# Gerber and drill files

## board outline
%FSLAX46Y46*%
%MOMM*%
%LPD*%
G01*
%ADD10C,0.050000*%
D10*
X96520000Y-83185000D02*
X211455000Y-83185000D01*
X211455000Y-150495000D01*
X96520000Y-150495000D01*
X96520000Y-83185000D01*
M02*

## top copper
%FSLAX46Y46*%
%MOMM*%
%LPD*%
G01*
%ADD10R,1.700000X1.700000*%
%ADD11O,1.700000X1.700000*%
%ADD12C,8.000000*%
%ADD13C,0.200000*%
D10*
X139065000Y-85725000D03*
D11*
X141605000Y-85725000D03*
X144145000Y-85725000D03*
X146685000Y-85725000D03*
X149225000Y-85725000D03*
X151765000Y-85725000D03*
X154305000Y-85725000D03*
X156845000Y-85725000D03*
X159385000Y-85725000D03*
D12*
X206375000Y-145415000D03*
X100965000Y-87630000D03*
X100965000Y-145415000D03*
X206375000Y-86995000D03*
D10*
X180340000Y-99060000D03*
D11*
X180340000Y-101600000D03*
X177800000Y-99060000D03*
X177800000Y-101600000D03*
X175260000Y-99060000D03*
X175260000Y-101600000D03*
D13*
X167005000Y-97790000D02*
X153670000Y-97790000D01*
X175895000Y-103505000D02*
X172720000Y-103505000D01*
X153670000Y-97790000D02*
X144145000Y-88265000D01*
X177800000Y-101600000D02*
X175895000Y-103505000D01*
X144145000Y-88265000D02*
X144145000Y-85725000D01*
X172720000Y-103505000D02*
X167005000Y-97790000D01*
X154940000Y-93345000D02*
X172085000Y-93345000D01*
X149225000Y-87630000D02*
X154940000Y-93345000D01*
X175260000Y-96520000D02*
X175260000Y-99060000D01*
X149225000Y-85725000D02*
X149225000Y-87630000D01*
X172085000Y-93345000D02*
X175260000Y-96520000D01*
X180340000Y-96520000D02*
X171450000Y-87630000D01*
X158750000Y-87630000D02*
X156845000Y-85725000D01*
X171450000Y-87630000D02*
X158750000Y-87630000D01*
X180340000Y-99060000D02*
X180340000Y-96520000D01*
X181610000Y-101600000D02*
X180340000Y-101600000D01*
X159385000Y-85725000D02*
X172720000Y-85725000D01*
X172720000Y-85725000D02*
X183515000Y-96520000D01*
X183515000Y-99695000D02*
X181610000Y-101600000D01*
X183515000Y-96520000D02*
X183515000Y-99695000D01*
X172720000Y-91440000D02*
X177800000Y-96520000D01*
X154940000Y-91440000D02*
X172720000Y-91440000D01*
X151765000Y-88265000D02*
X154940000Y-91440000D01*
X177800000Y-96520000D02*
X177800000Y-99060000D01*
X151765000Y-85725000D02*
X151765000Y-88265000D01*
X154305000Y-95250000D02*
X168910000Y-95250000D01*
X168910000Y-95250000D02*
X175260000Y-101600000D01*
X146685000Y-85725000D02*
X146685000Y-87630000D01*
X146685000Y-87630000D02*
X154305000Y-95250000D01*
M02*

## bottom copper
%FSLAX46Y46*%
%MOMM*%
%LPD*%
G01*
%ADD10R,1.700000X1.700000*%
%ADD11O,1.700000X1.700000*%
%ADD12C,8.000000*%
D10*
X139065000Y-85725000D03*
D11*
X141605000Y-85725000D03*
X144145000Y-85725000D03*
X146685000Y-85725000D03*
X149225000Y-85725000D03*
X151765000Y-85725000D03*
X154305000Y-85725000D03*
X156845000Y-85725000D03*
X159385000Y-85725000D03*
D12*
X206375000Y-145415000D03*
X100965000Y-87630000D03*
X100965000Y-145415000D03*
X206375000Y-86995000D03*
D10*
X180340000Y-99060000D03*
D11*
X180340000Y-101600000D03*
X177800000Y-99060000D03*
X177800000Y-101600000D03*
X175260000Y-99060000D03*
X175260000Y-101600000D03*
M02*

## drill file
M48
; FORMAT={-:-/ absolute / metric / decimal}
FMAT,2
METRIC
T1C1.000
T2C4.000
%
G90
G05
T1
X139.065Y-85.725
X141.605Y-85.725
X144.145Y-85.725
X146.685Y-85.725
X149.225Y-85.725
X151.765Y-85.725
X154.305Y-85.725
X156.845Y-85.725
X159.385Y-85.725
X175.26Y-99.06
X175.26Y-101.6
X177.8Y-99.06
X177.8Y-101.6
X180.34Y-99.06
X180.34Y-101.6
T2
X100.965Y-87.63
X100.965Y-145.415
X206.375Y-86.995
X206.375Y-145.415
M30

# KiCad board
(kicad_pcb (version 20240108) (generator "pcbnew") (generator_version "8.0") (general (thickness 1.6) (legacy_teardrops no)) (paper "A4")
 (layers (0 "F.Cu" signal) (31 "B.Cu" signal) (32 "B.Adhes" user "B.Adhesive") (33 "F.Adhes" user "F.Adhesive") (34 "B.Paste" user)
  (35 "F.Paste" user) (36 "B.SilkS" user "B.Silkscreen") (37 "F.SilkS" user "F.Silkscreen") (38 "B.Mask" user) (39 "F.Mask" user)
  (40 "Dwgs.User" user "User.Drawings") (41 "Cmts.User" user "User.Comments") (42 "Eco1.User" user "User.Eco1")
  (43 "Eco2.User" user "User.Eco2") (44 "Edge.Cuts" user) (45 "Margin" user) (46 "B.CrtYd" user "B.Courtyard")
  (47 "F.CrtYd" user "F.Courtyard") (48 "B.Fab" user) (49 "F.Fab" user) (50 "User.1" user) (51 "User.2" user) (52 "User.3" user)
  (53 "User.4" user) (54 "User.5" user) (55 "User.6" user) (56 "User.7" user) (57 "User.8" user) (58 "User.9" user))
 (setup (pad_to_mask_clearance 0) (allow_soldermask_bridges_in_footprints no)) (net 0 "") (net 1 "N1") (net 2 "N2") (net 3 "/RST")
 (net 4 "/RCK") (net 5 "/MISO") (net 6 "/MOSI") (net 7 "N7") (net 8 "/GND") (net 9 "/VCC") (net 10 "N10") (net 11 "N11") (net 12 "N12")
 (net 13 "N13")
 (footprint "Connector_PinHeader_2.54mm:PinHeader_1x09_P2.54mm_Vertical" (layer "F.Cu") (at 139.065 85.725 90)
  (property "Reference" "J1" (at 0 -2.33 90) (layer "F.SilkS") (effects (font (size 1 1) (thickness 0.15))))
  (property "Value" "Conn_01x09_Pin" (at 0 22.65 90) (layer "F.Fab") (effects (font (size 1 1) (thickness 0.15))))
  (pad "1" thru_hole rect (at 0 0 90) (size 1.7 1.7) (drill 1) (layers "*.Cu" "*.Mask") (remove_unused_layers no) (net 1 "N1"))
  (pad "2" thru_hole oval (at 0 2.54 90) (size 1.7 1.7) (drill 1) (layers "*.Cu" "*.Mask") (remove_unused_layers no) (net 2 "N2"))
  (pad "3" thru_hole oval (at 0 5.08 90) (size 1.7 1.7) (drill 1) (layers "*.Cu" "*.Mask") (remove_unused_layers no) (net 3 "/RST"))
  (pad "4" thru_hole oval (at 0 7.62 90) (size 1.7 1.7) (drill 1) (layers "*.Cu" "*.Mask") (remove_unused_layers no) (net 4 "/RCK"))
  (pad "5" thru_hole oval (at 0 10.16 90) (size 1.7 1.7) (drill 1) (layers "*.Cu" "*.Mask") (remove_unused_layers no) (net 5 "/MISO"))
  (pad "6" thru_hole oval (at 0 12.7 90) (size 1.7 1.7) (drill 1) (layers "*.Cu" "*.Mask") (remove_unused_layers no) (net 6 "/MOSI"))
  (pad "7" thru_hole oval (at 0 15.24 90) (size 1.7 1.7) (drill 1) (layers "*.Cu" "*.Mask") (remove_unused_layers no) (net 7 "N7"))
  (pad "8" thru_hole oval (at 0 17.78 90) (size 1.7 1.7) (drill 1) (layers "*.Cu" "*.Mask") (remove_unused_layers no) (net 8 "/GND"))
  (pad "9" thru_hole oval (at 0 20.32 90) (size 1.7 1.7) (drill 1) (layers "*.Cu" "*.Mask") (remove_unused_layers no) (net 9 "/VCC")))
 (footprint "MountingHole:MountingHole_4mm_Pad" (layer "F.Cu") (at 206.375 145.415 90)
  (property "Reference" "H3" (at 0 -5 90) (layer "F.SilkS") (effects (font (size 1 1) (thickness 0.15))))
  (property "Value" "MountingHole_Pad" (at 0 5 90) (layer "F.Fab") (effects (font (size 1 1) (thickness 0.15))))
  (pad "1" thru_hole circle (at 0 0 90) (size 8 8) (drill 4) (layers "*.Cu" "*.Mask") (remove_unused_layers no) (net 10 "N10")))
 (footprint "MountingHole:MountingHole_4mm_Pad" (layer "F.Cu") (at 100.965 87.63 90)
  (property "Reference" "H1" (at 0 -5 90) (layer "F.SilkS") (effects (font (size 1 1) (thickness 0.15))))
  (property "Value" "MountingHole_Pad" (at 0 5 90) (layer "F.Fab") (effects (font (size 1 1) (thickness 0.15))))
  (pad "1" thru_hole circle (at 0 0 90) (size 8 8) (drill 4) (layers "*.Cu" "*.Mask") (remove_unused_layers no) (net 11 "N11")))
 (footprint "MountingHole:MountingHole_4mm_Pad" (layer "F.Cu") (at 100.965 145.415 90)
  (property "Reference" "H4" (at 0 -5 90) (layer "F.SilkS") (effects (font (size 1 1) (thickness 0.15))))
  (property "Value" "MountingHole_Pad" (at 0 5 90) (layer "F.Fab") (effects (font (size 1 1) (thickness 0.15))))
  (pad "1" thru_hole circle (at 0 0 90) (size 8 8) (drill 4) (layers "*.Cu" "*.Mask") (remove_unused_layers no) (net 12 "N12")))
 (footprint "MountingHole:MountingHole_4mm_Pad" (layer "F.Cu") (at 206.375 86.995 90)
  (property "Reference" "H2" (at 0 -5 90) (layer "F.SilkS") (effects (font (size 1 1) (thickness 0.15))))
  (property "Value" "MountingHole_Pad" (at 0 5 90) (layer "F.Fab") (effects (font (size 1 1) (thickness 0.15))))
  (pad "1" thru_hole circle (at 0 0 90) (size 8 8) (drill 4) (layers "*.Cu" "*.Mask") (remove_unused_layers no) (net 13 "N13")))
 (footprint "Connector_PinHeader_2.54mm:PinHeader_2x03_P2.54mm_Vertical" (layer "F.Cu") (at 180.34 99.06 -90)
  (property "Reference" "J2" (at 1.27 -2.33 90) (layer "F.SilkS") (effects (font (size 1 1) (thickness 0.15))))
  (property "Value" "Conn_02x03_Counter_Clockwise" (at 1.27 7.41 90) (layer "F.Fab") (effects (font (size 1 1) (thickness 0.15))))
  (pad "1" thru_hole rect (at 0 0 270) (size 1.7 1.7) (drill 1) (layers "*.Cu" "*.Mask") (remove_unused_layers no) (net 8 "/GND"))
  (pad "2" thru_hole oval (at 2.54 0 270) (size 1.7 1.7) (drill 1) (layers "*.Cu" "*.Mask") (remove_unused_layers no) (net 9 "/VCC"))
  (pad "3" thru_hole oval (at 0 2.54 270) (size 1.7 1.7) (drill 1) (layers "*.Cu" "*.Mask") (remove_unused_layers no) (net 6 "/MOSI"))
  (pad "4" thru_hole oval (at 2.54 2.54 270) (size 1.7 1.7) (drill 1) (layers "*.Cu" "*.Mask") (remove_unused_layers no) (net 3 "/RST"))
  (pad "5" thru_hole oval (at 0 5.08 270) (size 1.7 1.7) (drill 1) (layers "*.Cu" "*.Mask") (remove_unused_layers no) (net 5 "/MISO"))
  (pad "6" thru_hole oval (at 2.54 5.08 270) (size 1.7 1.7) (drill 1) (layers "*.Cu" "*.Mask") (remove_unused_layers no) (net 4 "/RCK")))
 (gr_rect (start 96.52 83.185) (end 211.455 150.495) (stroke (width 0.05) (type default)) (fill none) (layer "Edge.Cuts"))
 (segment (start 167.005 97.79) (end 153.67 97.79) (width 0.2) (layer "F.Cu") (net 3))
 (segment (start 175.895 103.505) (end 172.72 103.505) (width 0.2) (layer "F.Cu") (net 3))
 (segment (start 153.67 97.79) (end 144.145 88.265) (width 0.2) (layer "F.Cu") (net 3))
 (segment (start 177.8 101.6) (end 175.895 103.505) (width 0.2) (layer "F.Cu") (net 3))
 (segment (start 144.145 88.265) (end 144.145 85.725) (width 0.2) (layer "F.Cu") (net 3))
 (segment (start 172.72 103.505) (end 167.005 97.79) (width 0.2) (layer "F.Cu") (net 3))
 (segment (start 154.94 93.345) (end 172.085 93.345) (width 0.2) (layer "F.Cu") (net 5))
 (segment (start 149.225 87.63) (end 154.94 93.345) (width 0.2) (layer "F.Cu") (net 5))
 (segment (start 175.26 96.52) (end 175.26 99.06) (width 0.2) (layer "F.Cu") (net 5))
 (segment (start 149.225 85.725) (end 149.225 87.63) (width 0.2) (layer "F.Cu") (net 5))
 (segment (start 172.085 93.345) (end 175.26 96.52) (width 0.2) (layer "F.Cu") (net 5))
 (segment (start 180.34 96.52) (end 171.45 87.63) (width 0.2) (layer "F.Cu") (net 8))
 (segment (start 158.75 87.63) (end 156.845 85.725) (width 0.2) (layer "F.Cu") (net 8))
 (segment (start 171.45 87.63) (end 158.75 87.63) (width 0.2) (layer "F.Cu") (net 8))
 (segment (start 180.34 99.06) (end 180.34 96.52) (width 0.2) (layer "F.Cu") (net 8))
 (segment (start 181.61 101.6) (end 180.34 101.6) (width 0.2) (layer "F.Cu") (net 9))
 (segment (start 159.385 85.725) (end 172.72 85.725) (width 0.2) (layer "F.Cu") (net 9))
 (segment (start 172.72 85.725) (end 183.515 96.52) (width 0.2) (layer "F.Cu") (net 9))
 (segment (start 183.515 99.695) (end 181.61 101.6) (width 0.2) (layer "F.Cu") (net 9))
 (segment (start 183.515 96.52) (end 183.515 99.695) (width 0.2) (layer "F.Cu") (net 9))
 (segment (start 172.72 91.44) (end 177.8 96.52) (width 0.2) (layer "F.Cu") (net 6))
 (segment (start 154.94 91.44) (end 172.72 91.44) (width 0.2) (layer "F.Cu") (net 6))
 (segment (start 151.765 88.265) (end 154.94 91.44) (width 0.2) (layer "F.Cu") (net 6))
 (segment (start 177.8 96.52) (end 177.8 99.06) (width 0.2) (layer "F.Cu") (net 6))
 (segment (start 151.765 85.725) (end 151.765 88.265) (width 0.2) (layer "F.Cu") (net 6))
 (segment (start 154.305 95.25) (end 168.91 95.25) (width 0.2) (layer "F.Cu") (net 4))
 (segment (start 168.91 95.25) (end 175.26 101.6) (width 0.2) (layer "F.Cu") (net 4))
 (segment (start 146.685 85.725) (end 146.685 87.63) (width 0.2) (layer "F.Cu") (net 4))
 (segment (start 146.685 87.63) (end 154.305 95.25) (width 0.2) (layer "F.Cu") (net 4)))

